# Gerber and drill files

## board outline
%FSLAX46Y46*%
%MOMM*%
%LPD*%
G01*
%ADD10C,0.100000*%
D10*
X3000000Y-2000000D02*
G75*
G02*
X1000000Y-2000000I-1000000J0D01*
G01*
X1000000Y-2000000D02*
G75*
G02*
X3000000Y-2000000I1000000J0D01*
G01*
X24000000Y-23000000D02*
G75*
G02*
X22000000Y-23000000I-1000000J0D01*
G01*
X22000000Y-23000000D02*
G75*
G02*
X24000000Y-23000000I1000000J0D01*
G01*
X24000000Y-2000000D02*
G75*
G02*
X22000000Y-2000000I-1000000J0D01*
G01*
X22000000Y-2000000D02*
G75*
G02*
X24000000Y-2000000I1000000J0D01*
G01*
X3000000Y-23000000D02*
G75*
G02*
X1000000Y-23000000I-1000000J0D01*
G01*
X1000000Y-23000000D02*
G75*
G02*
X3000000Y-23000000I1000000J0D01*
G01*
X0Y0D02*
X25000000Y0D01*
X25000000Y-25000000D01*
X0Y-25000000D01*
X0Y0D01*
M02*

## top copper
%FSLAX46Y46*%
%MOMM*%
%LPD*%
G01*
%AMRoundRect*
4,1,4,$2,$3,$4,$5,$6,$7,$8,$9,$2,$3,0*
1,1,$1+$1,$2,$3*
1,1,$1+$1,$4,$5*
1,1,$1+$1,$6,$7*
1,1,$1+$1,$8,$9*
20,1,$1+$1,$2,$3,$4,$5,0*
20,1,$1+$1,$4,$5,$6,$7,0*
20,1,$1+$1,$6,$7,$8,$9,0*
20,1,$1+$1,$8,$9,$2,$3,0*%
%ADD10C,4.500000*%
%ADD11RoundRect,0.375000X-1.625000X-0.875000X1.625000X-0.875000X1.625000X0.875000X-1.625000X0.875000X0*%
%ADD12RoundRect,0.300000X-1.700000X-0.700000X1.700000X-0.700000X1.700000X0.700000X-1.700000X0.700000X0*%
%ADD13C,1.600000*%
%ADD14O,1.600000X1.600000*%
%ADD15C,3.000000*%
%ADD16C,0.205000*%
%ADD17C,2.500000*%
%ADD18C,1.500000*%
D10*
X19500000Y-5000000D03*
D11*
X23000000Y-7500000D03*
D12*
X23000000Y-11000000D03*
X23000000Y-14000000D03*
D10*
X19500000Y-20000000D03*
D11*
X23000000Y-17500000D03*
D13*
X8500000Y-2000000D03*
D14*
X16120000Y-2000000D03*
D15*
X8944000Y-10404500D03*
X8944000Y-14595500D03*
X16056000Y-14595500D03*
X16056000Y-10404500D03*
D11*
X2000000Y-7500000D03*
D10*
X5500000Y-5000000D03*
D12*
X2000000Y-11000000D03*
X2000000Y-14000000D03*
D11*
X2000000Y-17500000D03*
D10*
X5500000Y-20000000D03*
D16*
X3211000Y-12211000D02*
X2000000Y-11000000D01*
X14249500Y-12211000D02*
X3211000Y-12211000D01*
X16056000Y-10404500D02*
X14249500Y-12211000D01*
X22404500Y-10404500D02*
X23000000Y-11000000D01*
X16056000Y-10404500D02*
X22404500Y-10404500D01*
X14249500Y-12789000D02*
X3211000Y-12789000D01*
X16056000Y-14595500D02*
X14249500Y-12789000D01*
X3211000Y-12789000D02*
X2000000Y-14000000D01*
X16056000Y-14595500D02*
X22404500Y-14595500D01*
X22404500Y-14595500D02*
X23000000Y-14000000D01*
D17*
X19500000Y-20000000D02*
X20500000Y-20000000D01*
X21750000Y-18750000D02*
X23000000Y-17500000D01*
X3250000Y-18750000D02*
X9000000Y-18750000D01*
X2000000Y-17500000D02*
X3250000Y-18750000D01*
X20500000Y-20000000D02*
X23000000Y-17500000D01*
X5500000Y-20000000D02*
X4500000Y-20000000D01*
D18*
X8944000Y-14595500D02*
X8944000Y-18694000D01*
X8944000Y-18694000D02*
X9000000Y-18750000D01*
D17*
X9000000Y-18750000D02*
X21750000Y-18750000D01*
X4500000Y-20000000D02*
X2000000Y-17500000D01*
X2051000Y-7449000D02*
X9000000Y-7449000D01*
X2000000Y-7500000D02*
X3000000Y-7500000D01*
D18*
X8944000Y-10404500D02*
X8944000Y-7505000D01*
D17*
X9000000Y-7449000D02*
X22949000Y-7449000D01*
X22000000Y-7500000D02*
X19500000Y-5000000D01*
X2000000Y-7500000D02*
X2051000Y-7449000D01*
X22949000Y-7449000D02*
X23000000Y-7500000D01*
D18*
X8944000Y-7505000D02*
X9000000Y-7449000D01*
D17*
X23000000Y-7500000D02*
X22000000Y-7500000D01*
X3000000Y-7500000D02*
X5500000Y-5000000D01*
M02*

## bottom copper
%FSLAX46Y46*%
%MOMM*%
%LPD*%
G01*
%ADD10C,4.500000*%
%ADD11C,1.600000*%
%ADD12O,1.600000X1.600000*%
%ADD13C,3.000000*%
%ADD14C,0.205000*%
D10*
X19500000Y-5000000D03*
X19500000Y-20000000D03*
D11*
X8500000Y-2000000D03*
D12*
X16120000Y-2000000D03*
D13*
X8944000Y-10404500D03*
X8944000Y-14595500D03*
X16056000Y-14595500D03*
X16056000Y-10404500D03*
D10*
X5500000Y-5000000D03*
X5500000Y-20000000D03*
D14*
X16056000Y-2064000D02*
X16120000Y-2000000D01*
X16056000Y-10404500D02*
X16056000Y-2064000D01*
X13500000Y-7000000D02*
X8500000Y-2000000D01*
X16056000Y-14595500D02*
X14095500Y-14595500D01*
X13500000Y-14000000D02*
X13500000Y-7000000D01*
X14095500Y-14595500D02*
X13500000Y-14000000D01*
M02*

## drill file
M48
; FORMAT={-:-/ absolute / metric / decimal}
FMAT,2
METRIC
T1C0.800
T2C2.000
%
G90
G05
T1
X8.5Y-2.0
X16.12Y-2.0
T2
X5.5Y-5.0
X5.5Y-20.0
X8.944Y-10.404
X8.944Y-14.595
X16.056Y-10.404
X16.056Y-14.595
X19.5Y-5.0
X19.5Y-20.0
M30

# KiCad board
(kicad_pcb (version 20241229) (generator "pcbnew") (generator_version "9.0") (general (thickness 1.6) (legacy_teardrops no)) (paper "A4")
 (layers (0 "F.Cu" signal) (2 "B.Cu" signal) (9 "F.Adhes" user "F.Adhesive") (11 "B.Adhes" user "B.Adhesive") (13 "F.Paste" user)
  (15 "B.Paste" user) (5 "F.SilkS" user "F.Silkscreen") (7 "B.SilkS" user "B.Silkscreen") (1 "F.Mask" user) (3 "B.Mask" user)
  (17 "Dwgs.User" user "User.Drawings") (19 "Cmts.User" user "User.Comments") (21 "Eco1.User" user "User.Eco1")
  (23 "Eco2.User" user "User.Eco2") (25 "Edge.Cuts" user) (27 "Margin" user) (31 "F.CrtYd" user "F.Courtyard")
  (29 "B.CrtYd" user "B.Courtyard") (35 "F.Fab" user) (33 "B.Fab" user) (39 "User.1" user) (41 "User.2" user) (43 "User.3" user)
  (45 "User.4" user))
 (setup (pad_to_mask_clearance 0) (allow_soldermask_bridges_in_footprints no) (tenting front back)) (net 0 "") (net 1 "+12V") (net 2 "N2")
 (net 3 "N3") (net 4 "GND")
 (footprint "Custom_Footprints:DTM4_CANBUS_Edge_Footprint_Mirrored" (layer "F.Cu") (at 23 12.5)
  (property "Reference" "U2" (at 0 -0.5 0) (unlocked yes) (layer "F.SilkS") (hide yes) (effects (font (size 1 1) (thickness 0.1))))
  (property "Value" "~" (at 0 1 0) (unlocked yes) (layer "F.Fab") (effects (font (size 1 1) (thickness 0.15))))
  (pad "1" thru_hole circle (at -3.5 -7.5) (size 4.5 4.5) (drill 2) (layers "*.Cu" "*.Mask") (remove_unused_layers no) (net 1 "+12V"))
  (pad "1" connect roundrect (at 0 -5) (size 4 2.5) (layers "F.Cu" "F.Mask") (roundrect_rratio 0.15) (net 1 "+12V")
   (thermal_bridge_angle 45))
  (pad "2" connect roundrect (at 0 -1.5) (size 4 2) (layers "F.Cu" "F.Mask") (roundrect_rratio 0.15) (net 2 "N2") (thermal_bridge_angle 45))
  (pad "3" connect roundrect (at 0 1.5) (size 4 2) (layers "F.Cu" "F.Mask") (roundrect_rratio 0.15) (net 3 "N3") (thermal_bridge_angle 45))
  (pad "4" thru_hole circle (at -3.5 7.5) (size 4.5 4.5) (drill 2) (layers "*.Cu" "*.Mask") (remove_unused_layers no) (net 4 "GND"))
  (pad "4" connect roundrect (at 0 5) (size 4 2.5) (layers "F.Cu" "F.Mask") (roundrect_rratio 0.15) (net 4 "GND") (thermal_bridge_angle 45)))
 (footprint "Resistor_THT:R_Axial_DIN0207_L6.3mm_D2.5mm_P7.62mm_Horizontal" (layer "F.Cu") (at 8.5 2)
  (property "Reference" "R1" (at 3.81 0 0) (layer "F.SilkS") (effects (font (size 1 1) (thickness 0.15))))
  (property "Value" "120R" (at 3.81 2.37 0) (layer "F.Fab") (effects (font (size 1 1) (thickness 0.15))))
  (pad "1" thru_hole circle (at 0 0) (size 1.6 1.6) (drill 0.8) (layers "*.Cu" "*.Mask") (remove_unused_layers no) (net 3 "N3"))
  (pad "2" thru_hole oval (at 7.62 0) (size 1.6 1.6) (drill 0.8) (layers "*.Cu" "*.Mask") (remove_unused_layers no) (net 2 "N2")))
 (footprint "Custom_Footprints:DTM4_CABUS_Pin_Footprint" (layer "F.Cu") (at 12.5 12.5)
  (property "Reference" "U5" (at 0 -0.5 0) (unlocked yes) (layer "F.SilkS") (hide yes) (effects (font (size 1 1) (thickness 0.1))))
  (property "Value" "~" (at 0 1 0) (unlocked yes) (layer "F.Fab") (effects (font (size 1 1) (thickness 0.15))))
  (pad "1" thru_hole circle (at -3.556 -2.0955) (size 3 3) (drill 2) (layers "*.Cu" "*.Mask") (remove_unused_layers no) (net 1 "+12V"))
  (pad "2" thru_hole circle (at -3.556 2.0955) (size 3 3) (drill 2) (layers "*.Cu" "*.Mask") (remove_unused_layers no) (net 4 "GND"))
  (pad "3" thru_hole circle (at 3.556 2.0955) (size 3 3) (drill 2) (layers "*.Cu" "*.Mask") (remove_unused_layers no) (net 3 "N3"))
  (pad "4" thru_hole circle (at 3.556 -2.0955) (size 3 3) (drill 2) (layers "*.Cu" "*.Mask") (remove_unused_layers no) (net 2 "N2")))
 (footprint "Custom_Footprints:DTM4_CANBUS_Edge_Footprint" (layer "F.Cu") (at 2 12.5)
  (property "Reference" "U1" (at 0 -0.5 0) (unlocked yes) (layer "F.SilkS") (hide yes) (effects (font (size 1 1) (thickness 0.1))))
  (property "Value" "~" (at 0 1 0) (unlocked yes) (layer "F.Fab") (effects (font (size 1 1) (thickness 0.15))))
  (pad "1" connect roundrect (at 0 -5) (size 4 2.5) (layers "F.Cu" "F.Mask") (roundrect_rratio 0.15) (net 1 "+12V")
   (thermal_bridge_angle 45))
  (pad "1" thru_hole circle (at 3.5 -7.5) (size 4.5 4.5) (drill 2) (layers "*.Cu" "*.Mask") (remove_unused_layers no) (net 1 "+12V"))
  (pad "2" connect roundrect (at 0 -1.5) (size 4 2) (layers "F.Cu" "F.Mask") (roundrect_rratio 0.15) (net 2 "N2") (thermal_bridge_angle 45))
  (pad "3" connect roundrect (at 0 1.5) (size 4 2) (layers "F.Cu" "F.Mask") (roundrect_rratio 0.15) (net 3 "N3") (thermal_bridge_angle 45))
  (pad "4" connect roundrect (at 0 5) (size 4 2.5) (layers "F.Cu" "F.Mask") (roundrect_rratio 0.15) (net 4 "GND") (thermal_bridge_angle 45))
  (pad "4" thru_hole circle (at 3.5 7.5) (size 4.5 4.5) (drill 2) (layers "*.Cu" "*.Mask") (remove_unused_layers no) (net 4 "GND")))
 (gr_circle (center 2 2) (end 3 2) (stroke (width 0.1) (type solid)) (fill no) (layer "Edge.Cuts"))
 (gr_circle (center 23 23) (end 24 23) (stroke (width 0.1) (type solid)) (fill no) (layer "Edge.Cuts"))
 (gr_circle (center 23 2) (end 24 2) (stroke (width 0.1) (type solid)) (fill no) (layer "Edge.Cuts"))
 (gr_circle (center 2 23) (end 3 23) (stroke (width 0.1) (type solid)) (fill no) (layer "Edge.Cuts"))
 (gr_rect (start 0 0) (end 25 25) (stroke (width 0.1) (type solid)) (fill no) (layer "Edge.Cuts"))
 (segment (start 3.211 12.211) (end 2 11) (width 0.205) (layer "F.Cu") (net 2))
 (segment (start 14.2495 12.211) (end 3.211 12.211) (width 0.205) (layer "F.Cu") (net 2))
 (segment (start 16.056 10.4045) (end 14.2495 12.211) (width 0.205) (layer "F.Cu") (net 2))
 (segment (start 22.4045 10.4045) (end 23 11) (width 0.205) (layer "F.Cu") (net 2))
 (segment (start 16.056 10.4045) (end 22.4045 10.4045) (width 0.205) (layer "F.Cu") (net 2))
 (segment (start 16.056 2.064) (end 16.12 2) (width 0.205) (layer "B.Cu") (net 2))
 (segment (start 16.056 10.4045) (end 16.056 2.064) (width 0.205) (layer "B.Cu") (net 2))
 (segment (start 14.2495 12.789) (end 3.211 12.789) (width 0.205) (layer "F.Cu") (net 3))
 (segment (start 16.056 14.5955) (end 14.2495 12.789) (width 0.205) (layer "F.Cu") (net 3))
 (segment (start 3.211 12.789) (end 2 14) (width 0.205) (layer "F.Cu") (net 3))
 (segment (start 16.056 14.5955) (end 22.4045 14.5955) (width 0.205) (layer "F.Cu") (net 3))
 (segment (start 22.4045 14.5955) (end 23 14) (width 0.205) (layer "F.Cu") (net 3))
 (segment (start 13.5 7) (end 8.5 2) (width 0.205) (layer "B.Cu") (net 3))
 (segment (start 16.056 14.5955) (end 14.0955 14.5955) (width 0.205) (layer "B.Cu") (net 3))
 (segment (start 13.5 14) (end 13.5 7) (width 0.205) (layer "B.Cu") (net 3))
 (segment (start 14.0955 14.5955) (end 13.5 14) (width 0.205) (layer "B.Cu") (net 3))
 (segment (start 19.5 20) (end 20.5 20) (width 2.5) (layer "F.Cu") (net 4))
 (segment (start 21.75 18.75) (end 23 17.5) (width 2.5) (layer "F.Cu") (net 4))
 (segment (start 3.25 18.75) (end 9 18.75) (width 2.5) (layer "F.Cu") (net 4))
 (segment (start 2 17.5) (end 3.25 18.75) (width 2.5) (layer "F.Cu") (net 4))
 (segment (start 20.5 20) (end 23 17.5) (width 2.5) (layer "F.Cu") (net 4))
 (segment (start 5.5 20) (end 4.5 20) (width 2.5) (layer "F.Cu") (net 4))
 (segment (start 8.944 14.5955) (end 8.944 18.694) (width 1.5) (layer "F.Cu") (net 4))
 (segment (start 8.944 18.694) (end 9 18.75) (width 1.5) (layer "F.Cu") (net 4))
 (segment (start 9 18.75) (end 21.75 18.75) (width 2.5) (layer "F.Cu") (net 4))
 (segment (start 4.5 20) (end 2 17.5) (width 2.5) (layer "F.Cu") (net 4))
 (segment (start 2.051 7.449) (end 9 7.449) (width 2.5) (layer "F.Cu") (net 1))
 (segment (start 2 7.5) (end 3 7.5) (width 2.5) (layer "F.Cu") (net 1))
 (segment (start 8.944 10.4045) (end 8.944 7.505) (width 1.5) (layer "F.Cu") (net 1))
 (segment (start 9 7.449) (end 22.949 7.449) (width 2.5) (layer "F.Cu") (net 1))
 (segment (start 22 7.5) (end 19.5 5) (width 2.5) (layer "F.Cu") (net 1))
 (segment (start 2 7.5) (end 2.051 7.449) (width 2.5) (layer "F.Cu") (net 1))
 (segment (start 22.949 7.449) (end 23 7.5) (width 2.5) (layer "F.Cu") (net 1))
 (segment (start 8.944 7.505) (end 9 7.449) (width 1.5) (layer "F.Cu") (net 1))
 (segment (start 23 7.5) (end 22 7.5) (width 2.5) (layer "F.Cu") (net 1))
 (segment (start 3 7.5) (end 5.5 5) (width 2.5) (layer "F.Cu") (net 1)))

